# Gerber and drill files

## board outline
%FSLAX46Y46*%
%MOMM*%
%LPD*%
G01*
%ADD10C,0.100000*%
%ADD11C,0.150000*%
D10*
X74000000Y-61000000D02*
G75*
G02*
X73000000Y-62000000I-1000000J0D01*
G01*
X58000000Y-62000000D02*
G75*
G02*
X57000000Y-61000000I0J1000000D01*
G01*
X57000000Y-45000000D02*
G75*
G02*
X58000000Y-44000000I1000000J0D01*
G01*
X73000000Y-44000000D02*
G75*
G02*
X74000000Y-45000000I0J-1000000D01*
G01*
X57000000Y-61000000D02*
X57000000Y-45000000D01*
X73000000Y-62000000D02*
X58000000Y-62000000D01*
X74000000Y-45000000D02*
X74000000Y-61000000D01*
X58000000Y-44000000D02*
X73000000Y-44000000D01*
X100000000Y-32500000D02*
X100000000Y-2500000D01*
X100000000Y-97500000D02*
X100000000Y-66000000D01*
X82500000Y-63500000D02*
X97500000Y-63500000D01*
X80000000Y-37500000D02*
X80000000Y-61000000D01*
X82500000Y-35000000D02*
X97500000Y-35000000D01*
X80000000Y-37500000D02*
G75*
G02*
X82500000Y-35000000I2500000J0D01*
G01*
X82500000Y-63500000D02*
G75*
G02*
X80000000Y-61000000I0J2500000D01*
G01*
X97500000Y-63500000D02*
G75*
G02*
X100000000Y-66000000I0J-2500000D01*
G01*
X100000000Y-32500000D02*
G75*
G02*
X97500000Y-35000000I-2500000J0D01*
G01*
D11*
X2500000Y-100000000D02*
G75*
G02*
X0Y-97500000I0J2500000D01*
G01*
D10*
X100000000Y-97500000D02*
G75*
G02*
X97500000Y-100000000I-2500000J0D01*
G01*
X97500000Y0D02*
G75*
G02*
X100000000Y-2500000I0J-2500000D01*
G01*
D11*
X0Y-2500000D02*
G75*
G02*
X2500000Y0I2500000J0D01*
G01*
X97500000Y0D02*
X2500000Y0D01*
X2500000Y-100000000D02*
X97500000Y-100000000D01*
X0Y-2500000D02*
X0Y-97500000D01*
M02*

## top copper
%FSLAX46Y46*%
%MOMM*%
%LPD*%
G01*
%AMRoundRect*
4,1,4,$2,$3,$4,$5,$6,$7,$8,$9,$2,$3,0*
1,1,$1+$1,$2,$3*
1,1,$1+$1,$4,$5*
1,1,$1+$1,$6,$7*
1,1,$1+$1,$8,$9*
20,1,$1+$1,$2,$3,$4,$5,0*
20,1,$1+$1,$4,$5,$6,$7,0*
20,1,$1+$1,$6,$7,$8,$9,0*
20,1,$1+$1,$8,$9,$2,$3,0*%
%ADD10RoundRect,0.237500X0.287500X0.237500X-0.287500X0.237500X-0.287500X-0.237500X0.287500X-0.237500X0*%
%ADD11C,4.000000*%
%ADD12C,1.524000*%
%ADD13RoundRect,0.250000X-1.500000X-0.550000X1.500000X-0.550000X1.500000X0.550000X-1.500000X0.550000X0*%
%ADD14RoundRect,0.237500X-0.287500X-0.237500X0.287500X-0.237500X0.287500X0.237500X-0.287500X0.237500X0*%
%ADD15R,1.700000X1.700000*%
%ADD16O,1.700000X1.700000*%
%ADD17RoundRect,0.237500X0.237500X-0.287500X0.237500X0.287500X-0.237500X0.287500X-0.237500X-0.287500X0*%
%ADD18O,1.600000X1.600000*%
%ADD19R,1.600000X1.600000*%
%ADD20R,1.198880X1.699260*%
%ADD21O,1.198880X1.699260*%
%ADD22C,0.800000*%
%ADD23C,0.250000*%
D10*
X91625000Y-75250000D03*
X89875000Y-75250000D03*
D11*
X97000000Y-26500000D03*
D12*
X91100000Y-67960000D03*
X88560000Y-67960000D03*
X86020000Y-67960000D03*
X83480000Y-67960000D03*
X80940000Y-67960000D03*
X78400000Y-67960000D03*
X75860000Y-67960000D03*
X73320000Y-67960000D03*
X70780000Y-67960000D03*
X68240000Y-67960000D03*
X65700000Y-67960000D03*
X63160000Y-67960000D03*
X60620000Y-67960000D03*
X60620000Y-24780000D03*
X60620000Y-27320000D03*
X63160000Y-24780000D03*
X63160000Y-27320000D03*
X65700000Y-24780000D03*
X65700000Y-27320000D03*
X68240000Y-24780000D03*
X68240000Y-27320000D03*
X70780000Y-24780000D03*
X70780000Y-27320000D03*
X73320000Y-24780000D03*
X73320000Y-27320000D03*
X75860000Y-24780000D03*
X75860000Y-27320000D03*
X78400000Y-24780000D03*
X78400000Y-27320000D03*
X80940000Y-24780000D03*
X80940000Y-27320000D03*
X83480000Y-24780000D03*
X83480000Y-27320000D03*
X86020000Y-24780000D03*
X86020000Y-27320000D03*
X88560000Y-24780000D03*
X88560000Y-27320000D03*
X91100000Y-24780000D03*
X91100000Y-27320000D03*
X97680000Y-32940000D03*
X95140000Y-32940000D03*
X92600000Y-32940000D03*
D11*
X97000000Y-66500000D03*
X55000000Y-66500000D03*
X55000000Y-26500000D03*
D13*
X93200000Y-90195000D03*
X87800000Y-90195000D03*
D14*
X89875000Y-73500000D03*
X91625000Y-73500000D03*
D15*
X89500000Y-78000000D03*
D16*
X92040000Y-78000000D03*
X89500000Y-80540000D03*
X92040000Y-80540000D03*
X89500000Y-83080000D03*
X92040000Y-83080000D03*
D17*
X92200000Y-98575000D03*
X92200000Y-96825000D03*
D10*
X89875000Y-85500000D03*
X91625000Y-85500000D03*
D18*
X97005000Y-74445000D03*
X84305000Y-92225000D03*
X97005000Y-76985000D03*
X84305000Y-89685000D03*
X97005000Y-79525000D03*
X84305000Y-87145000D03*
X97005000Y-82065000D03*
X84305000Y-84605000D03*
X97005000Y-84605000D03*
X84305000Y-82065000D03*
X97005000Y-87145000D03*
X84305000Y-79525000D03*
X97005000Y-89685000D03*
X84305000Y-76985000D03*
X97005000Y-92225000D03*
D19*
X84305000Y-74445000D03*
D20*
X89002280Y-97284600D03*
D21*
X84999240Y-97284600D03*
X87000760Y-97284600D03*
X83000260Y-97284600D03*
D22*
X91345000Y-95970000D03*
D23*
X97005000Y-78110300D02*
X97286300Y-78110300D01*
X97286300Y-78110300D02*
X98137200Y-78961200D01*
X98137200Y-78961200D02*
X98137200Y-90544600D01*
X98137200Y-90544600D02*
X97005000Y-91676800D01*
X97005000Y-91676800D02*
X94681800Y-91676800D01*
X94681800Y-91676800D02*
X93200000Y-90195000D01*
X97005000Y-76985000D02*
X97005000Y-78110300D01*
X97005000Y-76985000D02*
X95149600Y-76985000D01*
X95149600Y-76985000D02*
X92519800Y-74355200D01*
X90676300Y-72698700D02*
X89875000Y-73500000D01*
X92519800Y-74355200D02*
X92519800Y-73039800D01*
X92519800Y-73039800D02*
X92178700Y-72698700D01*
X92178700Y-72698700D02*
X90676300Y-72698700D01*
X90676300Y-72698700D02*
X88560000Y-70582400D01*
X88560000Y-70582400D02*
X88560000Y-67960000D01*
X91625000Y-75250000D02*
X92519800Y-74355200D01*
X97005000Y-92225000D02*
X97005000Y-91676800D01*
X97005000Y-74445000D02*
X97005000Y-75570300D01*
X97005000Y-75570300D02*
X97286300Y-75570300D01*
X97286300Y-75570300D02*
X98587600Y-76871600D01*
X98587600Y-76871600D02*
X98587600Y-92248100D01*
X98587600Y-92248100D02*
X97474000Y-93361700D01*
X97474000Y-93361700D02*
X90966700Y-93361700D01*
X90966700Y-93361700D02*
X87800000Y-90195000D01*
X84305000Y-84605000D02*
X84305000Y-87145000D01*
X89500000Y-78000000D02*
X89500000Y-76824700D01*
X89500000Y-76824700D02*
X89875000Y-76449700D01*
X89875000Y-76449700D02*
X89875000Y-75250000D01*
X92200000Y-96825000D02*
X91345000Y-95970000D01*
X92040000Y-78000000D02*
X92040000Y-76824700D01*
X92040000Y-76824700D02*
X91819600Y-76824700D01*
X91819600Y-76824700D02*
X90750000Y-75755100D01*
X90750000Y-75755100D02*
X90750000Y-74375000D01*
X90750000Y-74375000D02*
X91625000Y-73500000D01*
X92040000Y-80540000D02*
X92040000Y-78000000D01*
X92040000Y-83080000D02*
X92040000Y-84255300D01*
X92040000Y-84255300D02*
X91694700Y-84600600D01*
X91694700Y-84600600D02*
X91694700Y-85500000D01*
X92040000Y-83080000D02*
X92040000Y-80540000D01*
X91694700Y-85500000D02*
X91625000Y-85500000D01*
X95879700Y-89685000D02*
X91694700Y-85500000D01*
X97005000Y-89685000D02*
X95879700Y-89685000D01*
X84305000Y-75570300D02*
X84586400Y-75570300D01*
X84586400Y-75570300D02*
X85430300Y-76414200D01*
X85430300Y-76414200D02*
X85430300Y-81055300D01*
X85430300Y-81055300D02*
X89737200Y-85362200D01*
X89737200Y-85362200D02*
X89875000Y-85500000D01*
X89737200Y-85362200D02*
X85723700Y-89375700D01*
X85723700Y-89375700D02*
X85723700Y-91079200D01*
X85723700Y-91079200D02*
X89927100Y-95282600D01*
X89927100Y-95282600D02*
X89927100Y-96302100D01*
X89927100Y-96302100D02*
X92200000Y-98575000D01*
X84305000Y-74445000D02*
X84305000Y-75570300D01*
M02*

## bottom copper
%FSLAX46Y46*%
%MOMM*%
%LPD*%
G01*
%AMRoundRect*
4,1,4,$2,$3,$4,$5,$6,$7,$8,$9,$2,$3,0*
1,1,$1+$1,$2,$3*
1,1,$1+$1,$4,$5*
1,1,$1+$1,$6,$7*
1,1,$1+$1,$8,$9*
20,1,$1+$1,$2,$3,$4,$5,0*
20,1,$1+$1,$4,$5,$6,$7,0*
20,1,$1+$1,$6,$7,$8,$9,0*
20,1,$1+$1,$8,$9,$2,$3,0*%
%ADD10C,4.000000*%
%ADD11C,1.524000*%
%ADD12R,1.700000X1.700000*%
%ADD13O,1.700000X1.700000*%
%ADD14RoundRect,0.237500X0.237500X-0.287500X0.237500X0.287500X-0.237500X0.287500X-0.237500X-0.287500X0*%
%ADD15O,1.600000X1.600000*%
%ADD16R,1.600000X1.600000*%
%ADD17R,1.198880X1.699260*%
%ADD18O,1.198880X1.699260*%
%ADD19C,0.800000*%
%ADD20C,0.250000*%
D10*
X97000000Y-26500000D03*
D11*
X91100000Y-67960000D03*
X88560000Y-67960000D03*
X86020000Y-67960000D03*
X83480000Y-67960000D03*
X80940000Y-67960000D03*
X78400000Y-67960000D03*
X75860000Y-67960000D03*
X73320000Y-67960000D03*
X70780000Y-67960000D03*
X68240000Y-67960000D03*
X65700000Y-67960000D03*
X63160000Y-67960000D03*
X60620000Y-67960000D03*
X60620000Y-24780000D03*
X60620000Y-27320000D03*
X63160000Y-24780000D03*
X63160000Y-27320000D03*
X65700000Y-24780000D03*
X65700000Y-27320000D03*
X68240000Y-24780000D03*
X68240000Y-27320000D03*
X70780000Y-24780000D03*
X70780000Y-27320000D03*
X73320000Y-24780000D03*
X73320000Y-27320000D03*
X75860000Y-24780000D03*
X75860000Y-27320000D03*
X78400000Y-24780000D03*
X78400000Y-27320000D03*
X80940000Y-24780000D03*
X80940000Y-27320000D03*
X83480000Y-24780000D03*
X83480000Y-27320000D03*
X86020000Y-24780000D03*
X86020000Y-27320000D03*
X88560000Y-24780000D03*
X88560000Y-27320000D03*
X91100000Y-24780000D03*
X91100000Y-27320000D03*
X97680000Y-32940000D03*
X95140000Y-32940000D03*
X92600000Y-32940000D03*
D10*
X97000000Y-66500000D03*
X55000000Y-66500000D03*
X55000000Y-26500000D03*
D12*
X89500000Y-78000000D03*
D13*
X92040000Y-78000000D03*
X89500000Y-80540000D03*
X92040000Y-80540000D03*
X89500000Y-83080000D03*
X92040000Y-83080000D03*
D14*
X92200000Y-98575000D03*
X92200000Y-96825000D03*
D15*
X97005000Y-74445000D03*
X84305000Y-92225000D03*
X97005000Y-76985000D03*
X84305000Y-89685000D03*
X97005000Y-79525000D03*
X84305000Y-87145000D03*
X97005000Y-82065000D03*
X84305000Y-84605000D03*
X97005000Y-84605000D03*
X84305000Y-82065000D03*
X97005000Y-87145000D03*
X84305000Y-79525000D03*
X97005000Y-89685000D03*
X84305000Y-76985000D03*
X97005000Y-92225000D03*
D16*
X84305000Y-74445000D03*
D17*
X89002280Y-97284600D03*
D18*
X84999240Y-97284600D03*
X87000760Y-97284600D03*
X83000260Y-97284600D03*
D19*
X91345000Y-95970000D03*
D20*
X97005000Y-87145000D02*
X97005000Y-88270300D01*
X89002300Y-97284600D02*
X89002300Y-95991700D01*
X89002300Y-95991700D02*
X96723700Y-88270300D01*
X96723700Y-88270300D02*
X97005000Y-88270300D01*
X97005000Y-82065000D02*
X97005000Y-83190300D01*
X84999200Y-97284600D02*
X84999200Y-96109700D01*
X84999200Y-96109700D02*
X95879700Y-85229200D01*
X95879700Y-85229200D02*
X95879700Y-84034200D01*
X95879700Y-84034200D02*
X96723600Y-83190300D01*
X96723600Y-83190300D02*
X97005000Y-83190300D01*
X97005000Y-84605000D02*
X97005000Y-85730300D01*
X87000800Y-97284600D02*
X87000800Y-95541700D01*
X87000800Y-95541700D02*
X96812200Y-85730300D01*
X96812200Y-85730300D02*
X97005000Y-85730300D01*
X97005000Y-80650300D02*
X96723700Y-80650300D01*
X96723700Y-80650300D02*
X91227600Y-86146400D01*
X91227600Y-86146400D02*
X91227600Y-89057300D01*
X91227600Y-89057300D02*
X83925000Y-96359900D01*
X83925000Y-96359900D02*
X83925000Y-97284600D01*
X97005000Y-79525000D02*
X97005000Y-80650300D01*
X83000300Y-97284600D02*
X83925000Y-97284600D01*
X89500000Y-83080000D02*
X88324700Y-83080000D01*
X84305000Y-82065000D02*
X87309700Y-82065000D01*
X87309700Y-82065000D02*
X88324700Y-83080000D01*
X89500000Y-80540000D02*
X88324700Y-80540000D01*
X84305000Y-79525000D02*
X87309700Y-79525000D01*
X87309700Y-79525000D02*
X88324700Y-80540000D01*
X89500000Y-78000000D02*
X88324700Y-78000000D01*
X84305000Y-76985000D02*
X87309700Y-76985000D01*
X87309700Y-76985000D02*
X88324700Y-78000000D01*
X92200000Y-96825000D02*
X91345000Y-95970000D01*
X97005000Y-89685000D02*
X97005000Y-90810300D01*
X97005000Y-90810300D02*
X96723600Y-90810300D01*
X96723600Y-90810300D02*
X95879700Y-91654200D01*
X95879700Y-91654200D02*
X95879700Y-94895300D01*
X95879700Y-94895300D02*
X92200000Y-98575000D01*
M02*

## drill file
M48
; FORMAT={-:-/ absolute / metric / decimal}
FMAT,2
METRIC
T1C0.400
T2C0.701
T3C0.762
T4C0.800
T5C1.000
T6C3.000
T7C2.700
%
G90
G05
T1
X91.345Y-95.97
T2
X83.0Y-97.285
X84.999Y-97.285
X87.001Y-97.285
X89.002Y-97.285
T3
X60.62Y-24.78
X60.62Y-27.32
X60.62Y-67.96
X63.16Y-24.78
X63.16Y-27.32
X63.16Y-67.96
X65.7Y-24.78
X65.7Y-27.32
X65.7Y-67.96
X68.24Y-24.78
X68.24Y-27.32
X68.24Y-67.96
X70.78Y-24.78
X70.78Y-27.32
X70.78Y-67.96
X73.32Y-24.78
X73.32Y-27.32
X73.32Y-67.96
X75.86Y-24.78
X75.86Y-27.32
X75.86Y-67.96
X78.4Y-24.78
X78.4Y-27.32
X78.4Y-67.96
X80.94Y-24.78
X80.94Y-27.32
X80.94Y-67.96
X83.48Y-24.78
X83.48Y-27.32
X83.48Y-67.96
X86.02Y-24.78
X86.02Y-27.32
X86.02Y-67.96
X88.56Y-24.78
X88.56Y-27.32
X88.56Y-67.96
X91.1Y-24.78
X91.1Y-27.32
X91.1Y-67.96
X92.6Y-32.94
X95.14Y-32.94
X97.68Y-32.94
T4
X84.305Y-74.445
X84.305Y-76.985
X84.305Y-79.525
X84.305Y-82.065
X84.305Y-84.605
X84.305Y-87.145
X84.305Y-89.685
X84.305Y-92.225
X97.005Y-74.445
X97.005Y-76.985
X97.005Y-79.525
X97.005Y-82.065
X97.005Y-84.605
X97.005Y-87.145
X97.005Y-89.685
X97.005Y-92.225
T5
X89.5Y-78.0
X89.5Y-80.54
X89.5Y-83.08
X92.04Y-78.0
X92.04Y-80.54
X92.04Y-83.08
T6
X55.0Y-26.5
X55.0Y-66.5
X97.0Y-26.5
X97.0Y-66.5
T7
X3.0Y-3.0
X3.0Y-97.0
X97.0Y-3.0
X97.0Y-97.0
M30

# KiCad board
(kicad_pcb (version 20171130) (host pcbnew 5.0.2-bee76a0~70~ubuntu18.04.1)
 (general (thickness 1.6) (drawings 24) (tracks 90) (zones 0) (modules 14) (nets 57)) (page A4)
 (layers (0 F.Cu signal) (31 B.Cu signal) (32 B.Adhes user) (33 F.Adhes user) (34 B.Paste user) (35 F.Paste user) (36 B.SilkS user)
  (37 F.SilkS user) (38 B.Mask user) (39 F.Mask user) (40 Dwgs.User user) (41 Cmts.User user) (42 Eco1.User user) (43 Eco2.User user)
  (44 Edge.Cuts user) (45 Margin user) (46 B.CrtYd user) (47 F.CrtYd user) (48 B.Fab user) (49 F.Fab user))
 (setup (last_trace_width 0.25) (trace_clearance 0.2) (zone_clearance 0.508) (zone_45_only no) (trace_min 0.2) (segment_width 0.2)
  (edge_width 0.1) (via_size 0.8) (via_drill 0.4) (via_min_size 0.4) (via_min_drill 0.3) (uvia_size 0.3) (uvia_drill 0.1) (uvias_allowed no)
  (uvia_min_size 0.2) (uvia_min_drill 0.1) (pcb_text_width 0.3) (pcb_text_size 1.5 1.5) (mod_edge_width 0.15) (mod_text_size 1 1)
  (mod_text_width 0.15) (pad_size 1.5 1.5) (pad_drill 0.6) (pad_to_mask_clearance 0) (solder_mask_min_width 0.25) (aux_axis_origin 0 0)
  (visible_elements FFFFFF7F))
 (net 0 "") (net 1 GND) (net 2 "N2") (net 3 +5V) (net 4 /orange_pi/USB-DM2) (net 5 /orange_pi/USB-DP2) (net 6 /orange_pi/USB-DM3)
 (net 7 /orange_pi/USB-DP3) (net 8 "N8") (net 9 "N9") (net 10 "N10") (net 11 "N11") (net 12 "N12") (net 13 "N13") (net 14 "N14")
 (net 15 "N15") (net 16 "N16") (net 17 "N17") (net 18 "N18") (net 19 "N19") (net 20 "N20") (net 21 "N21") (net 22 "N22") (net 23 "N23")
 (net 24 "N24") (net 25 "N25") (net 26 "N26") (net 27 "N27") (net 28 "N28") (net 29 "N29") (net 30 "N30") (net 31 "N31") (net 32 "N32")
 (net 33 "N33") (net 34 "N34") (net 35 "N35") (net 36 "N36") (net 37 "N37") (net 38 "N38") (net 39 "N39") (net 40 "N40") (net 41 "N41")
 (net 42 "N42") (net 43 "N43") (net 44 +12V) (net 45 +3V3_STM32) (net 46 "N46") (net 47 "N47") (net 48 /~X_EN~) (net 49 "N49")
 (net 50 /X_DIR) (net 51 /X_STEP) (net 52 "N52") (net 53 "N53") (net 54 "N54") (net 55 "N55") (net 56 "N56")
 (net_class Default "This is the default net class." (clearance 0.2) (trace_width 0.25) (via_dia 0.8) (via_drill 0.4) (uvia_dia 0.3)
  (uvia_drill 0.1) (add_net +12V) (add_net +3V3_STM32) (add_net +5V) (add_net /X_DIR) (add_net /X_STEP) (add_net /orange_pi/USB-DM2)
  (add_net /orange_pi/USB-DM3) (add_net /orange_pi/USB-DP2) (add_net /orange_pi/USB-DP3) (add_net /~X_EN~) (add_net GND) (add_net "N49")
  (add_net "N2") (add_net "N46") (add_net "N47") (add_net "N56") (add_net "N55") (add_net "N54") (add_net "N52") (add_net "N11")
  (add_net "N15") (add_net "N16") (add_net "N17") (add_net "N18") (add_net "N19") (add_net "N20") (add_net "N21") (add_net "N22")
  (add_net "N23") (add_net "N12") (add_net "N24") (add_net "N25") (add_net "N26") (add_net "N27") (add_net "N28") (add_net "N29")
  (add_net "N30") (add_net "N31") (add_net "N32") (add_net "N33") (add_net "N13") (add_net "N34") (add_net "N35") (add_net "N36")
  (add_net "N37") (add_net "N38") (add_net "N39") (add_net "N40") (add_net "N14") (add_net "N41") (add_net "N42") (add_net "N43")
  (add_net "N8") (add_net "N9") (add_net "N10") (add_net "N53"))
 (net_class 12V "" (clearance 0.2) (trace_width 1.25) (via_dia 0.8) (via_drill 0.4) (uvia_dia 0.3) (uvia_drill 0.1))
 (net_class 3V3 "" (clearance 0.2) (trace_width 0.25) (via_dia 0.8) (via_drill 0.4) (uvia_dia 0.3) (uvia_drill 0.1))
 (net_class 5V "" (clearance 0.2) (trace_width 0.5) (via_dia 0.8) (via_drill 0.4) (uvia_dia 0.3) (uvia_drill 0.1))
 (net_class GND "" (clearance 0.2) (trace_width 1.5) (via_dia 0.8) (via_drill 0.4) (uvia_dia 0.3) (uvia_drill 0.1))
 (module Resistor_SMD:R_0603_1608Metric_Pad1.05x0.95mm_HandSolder (layer F.Cu) (at 90.75 75.25 180)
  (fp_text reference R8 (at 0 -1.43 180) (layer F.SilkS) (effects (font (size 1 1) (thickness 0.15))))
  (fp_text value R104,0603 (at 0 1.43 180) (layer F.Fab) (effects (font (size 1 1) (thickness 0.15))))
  (pad 1 smd roundrect (at -0.875 0 180) (size 1.05 0.95) (layers F.Cu F.Paste F.Mask) (roundrect_rratio 0.25) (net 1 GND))
  (pad 2 smd roundrect (at 0.875 0 180) (size 1.05 0.95) (layers F.Cu F.Paste F.Mask) (roundrect_rratio 0.25) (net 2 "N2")))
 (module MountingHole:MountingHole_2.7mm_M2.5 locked (layer F.Cu) (at 3 97)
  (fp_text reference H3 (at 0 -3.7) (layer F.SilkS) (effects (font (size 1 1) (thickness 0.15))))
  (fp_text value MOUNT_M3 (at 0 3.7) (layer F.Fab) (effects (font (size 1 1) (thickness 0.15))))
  (pad 1 np_thru_hole circle (at 0 0) (size 2.7 2.7) (drill 2.7) (layers *.Cu *.Mask)))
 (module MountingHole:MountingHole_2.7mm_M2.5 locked (layer F.Cu) (at 97 97)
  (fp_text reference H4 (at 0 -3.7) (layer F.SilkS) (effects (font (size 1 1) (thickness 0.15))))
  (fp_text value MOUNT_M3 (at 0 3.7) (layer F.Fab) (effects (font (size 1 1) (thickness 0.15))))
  (pad 1 np_thru_hole circle (at 0 0) (size 2.7 2.7) (drill 2.7) (layers *.Cu *.Mask)))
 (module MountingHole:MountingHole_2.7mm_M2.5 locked (layer F.Cu) (at 3 3)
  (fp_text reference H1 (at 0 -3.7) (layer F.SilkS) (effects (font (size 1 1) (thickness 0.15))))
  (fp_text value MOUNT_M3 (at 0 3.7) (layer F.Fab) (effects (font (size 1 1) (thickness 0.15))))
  (pad 1 np_thru_hole circle (at 0 0) (size 2.7 2.7) (drill 2.7) (layers *.Cu *.Mask)))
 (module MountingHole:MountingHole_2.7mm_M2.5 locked (layer F.Cu) (at 97 3)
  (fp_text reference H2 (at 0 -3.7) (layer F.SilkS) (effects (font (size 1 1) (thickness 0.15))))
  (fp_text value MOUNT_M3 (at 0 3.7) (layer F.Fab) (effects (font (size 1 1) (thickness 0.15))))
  (pad 1 np_thru_hole circle (at 0 0) (size 2.7 2.7) (drill 2.7) (layers *.Cu *.Mask)))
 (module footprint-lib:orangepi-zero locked (layer B.Cu) (at 52 69.5 90)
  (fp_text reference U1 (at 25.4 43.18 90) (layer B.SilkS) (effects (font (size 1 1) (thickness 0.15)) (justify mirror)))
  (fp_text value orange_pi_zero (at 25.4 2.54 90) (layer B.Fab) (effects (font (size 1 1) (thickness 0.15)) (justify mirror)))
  (pad "" thru_hole circle (at 43 45 90) (size 4 4) (drill 3) (layers *.Cu *.Mask B.SilkS))
  (pad 1 thru_hole circle (at 1.54 39.1 90) (size 1.524 1.524) (drill 0.762) (layers *.Cu *.Mask B.SilkS) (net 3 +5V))
  (pad 2 thru_hole circle (at 1.54 36.56 90) (size 1.524 1.524) (drill 0.762) (layers *.Cu *.Mask B.SilkS) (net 1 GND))
  (pad 3 thru_hole circle (at 1.54 34.02 90) (size 1.524 1.524) (drill 0.762) (layers *.Cu *.Mask B.SilkS) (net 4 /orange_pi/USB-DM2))
  (pad 4 thru_hole circle (at 1.54 31.48 90) (size 1.524 1.524) (drill 0.762) (layers *.Cu *.Mask B.SilkS) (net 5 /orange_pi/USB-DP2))
  (pad 5 thru_hole circle (at 1.54 28.94 90) (size 1.524 1.524) (drill 0.762) (layers *.Cu *.Mask B.SilkS) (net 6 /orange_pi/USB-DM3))
  (pad 6 thru_hole circle (at 1.54 26.4 90) (size 1.524 1.524) (drill 0.762) (layers *.Cu *.Mask B.SilkS) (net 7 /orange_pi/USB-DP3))
  (pad 7 thru_hole circle (at 1.54 23.86 90) (size 1.524 1.524) (drill 0.762) (layers *.Cu *.Mask B.SilkS) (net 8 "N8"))
  (pad 8 thru_hole circle (at 1.54 21.32 90) (size 1.524 1.524) (drill 0.762) (layers *.Cu *.Mask B.SilkS) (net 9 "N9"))
  (pad 9 thru_hole circle (at 1.54 18.78 90) (size 1.524 1.524) (drill 0.762) (layers *.Cu *.Mask B.SilkS) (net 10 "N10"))
  (pad 10 thru_hole circle (at 1.54 16.24 90) (size 1.524 1.524) (drill 0.762) (layers *.Cu *.Mask B.SilkS) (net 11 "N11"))
  (pad 11 thru_hole circle (at 1.54 13.7 90) (size 1.524 1.524) (drill 0.762) (layers *.Cu *.Mask B.SilkS) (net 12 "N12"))
  (pad 12 thru_hole circle (at 1.54 11.16 90) (size 1.524 1.524) (drill 0.762) (layers *.Cu *.Mask B.SilkS) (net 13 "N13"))
  (pad 13 thru_hole circle (at 1.54 8.62 90) (size 1.524 1.524) (drill 0.762) (layers *.Cu *.Mask B.SilkS) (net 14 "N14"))
  (pad 101 thru_hole circle (at 44.72 8.62 90) (size 1.524 1.524) (drill 0.762) (layers *.Cu *.Mask B.SilkS) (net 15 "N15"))
  (pad 102 thru_hole circle (at 42.18 8.62 90) (size 1.524 1.524) (drill 0.762) (layers *.Cu *.Mask B.SilkS) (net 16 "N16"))
  (pad 103 thru_hole circle (at 44.72 11.16 90) (size 1.524 1.524) (drill 0.762) (layers *.Cu *.Mask B.SilkS) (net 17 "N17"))
  (pad 104 thru_hole circle (at 42.18 11.16 90) (size 1.524 1.524) (drill 0.762) (layers *.Cu *.Mask B.SilkS) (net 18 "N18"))
  (pad 105 thru_hole circle (at 44.72 13.7 90) (size 1.524 1.524) (drill 0.762) (layers *.Cu *.Mask B.SilkS) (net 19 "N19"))
  (pad 106 thru_hole circle (at 42.18 13.7 90) (size 1.524 1.524) (drill 0.762) (layers *.Cu *.Mask B.SilkS) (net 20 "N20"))
  (pad 107 thru_hole circle (at 44.72 16.24 90) (size 1.524 1.524) (drill 0.762) (layers *.Cu *.Mask B.SilkS) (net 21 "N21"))
  (pad 108 thru_hole circle (at 42.18 16.24 90) (size 1.524 1.524) (drill 0.762) (layers *.Cu *.Mask B.SilkS) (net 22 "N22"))
  (pad 109 thru_hole circle (at 44.72 18.78 90) (size 1.524 1.524) (drill 0.762) (layers *.Cu *.Mask B.SilkS) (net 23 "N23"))
  (pad 110 thru_hole circle (at 42.18 18.78 90) (size 1.524 1.524) (drill 0.762) (layers *.Cu *.Mask B.SilkS) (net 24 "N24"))
  (pad 111 thru_hole circle (at 44.72 21.32 90) (size 1.524 1.524) (drill 0.762) (layers *.Cu *.Mask B.SilkS) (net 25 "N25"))
  (pad 112 thru_hole circle (at 42.18 21.32 90) (size 1.524 1.524) (drill 0.762) (layers *.Cu *.Mask B.SilkS) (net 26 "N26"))
  (pad 113 thru_hole circle (at 44.72 23.86 90) (size 1.524 1.524) (drill 0.762) (layers *.Cu *.Mask B.SilkS) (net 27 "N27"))
  (pad 114 thru_hole circle (at 42.18 23.86 90) (size 1.524 1.524) (drill 0.762) (layers *.Cu *.Mask B.SilkS) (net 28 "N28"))
  (pad 115 thru_hole circle (at 44.72 26.4 90) (size 1.524 1.524) (drill 0.762) (layers *.Cu *.Mask B.SilkS) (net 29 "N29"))
  (pad 116 thru_hole circle (at 42.18 26.4 90) (size 1.524 1.524) (drill 0.762) (layers *.Cu *.Mask B.SilkS) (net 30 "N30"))
  (pad 117 thru_hole circle (at 44.72 28.94 90) (size 1.524 1.524) (drill 0.762) (layers *.Cu *.Mask B.SilkS) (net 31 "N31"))
  (pad 118 thru_hole circle (at 42.18 28.94 90) (size 1.524 1.524) (drill 0.762) (layers *.Cu *.Mask B.SilkS) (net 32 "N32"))
  (pad 119 thru_hole circle (at 44.72 31.48 90) (size 1.524 1.524) (drill 0.762) (layers *.Cu *.Mask B.SilkS) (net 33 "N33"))
  (pad 120 thru_hole circle (at 42.18 31.48 90) (size 1.524 1.524) (drill 0.762) (layers *.Cu *.Mask B.SilkS) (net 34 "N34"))
  (pad 121 thru_hole circle (at 44.72 34.02 90) (size 1.524 1.524) (drill 0.762) (layers *.Cu *.Mask B.SilkS) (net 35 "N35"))
  (pad 122 thru_hole circle (at 42.18 34.02 90) (size 1.524 1.524) (drill 0.762) (layers *.Cu *.Mask B.SilkS) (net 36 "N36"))
  (pad 123 thru_hole circle (at 44.72 36.56 90) (size 1.524 1.524) (drill 0.762) (layers *.Cu *.Mask B.SilkS) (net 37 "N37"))
  (pad 124 thru_hole circle (at 42.18 36.56 90) (size 1.524 1.524) (drill 0.762) (layers *.Cu *.Mask B.SilkS) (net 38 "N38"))
  (pad 125 thru_hole circle (at 44.72 39.1 90) (size 1.524 1.524) (drill 0.762) (layers *.Cu *.Mask B.SilkS) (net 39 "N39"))
  (pad 126 thru_hole circle (at 42.18 39.1 90) (size 1.524 1.524) (drill 0.762) (layers *.Cu *.Mask B.SilkS) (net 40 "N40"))
  (pad 201 thru_hole circle (at 36.56 45.68 90) (size 1.524 1.524) (drill 0.762) (layers *.Cu *.Mask B.SilkS) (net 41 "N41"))
  (pad 202 thru_hole circle (at 36.56 43.14 90) (size 1.524 1.524) (drill 0.762) (layers *.Cu *.Mask B.SilkS) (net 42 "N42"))
  (pad 203 thru_hole circle (at 36.56 40.6 90) (size 1.524 1.524) (drill 0.762) (layers *.Cu *.Mask B.SilkS) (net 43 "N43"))
  (pad "" thru_hole circle (at 3 45 90) (size 4 4) (drill 3) (layers *.Cu *.Mask B.SilkS))
  (pad "" thru_hole circle (at 3 3 90) (size 4 4) (drill 3) (layers *.Cu *.Mask B.SilkS))
  (pad "" thru_hole circle (at 43 3 90) (size 4 4) (drill 3) (layers *.Cu *.Mask B.SilkS)))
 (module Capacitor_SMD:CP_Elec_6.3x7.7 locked (layer F.Cu) (at 90.5 90.195)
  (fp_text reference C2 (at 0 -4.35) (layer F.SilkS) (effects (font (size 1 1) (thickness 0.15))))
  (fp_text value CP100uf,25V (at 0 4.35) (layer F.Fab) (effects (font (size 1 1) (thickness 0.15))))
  (pad 2 smd roundrect (at 2.7 0) (size 3.5 1.6) (layers F.Cu F.Paste F.Mask) (roundrect_rratio 0.15625) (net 1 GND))
  (pad 1 smd roundrect (at -2.7 0) (size 3.5 1.6) (layers F.Cu F.Paste F.Mask) (roundrect_rratio 0.15625) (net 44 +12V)))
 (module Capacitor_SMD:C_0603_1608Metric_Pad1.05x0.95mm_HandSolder (layer F.Cu) (at 90.75 73.5)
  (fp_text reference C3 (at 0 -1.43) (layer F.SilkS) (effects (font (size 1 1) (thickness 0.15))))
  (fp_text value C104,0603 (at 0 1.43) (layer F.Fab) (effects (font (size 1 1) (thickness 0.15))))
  (pad 1 smd roundrect (at -0.875 0) (size 1.05 0.95) (layers F.Cu F.Paste F.Mask) (roundrect_rratio 0.25) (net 1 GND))
  (pad 2 smd roundrect (at 0.875 0) (size 1.05 0.95) (layers F.Cu F.Paste F.Mask) (roundrect_rratio 0.25) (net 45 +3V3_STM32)))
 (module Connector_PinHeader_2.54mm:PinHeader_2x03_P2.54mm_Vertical (layer F.Cu) (at 89.5 78)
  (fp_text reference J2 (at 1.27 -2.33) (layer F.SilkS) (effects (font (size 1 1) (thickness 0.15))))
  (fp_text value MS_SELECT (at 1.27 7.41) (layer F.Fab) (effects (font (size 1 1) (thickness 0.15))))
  (pad 1 thru_hole rect (at 0 0) (size 1.7 1.7) (drill 1) (layers *.Cu *.Mask) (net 2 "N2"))
  (pad 2 thru_hole oval (at 2.54 0) (size 1.7 1.7) (drill 1) (layers *.Cu *.Mask) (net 45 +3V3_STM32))
  (pad 3 thru_hole oval (at 0 2.54) (size 1.7 1.7) (drill 1) (layers *.Cu *.Mask) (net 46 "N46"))
  (pad 4 thru_hole oval (at 2.54 2.54) (size 1.7 1.7) (drill 1) (layers *.Cu *.Mask) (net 45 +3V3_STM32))
  (pad 5 thru_hole oval (at 0 5.08) (size 1.7 1.7) (drill 1) (layers *.Cu *.Mask) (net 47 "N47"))
  (pad 6 thru_hole oval (at 2.54 5.08) (size 1.7 1.7) (drill 1) (layers *.Cu *.Mask) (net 45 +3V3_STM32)))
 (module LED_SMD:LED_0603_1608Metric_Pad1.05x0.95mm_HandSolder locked (layer F.Cu) (at 92.2 97.7 90)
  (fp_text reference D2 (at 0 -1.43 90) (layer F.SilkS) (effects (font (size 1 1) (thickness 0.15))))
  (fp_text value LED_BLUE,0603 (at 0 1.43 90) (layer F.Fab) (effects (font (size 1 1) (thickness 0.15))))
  (pad 1 smd roundrect (at -0.875 0 90) (size 1.05 0.95) (layers F.Cu F.Paste F.Mask) (roundrect_rratio 0.25) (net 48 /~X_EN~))
  (pad 2 smd roundrect (at 0.875 0 90) (size 1.05 0.95) (layers F.Cu F.Paste F.Mask) (roundrect_rratio 0.25) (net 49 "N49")))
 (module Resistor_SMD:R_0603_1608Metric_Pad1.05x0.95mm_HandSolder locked (layer B.Cu) (at 92.2 97.7 90)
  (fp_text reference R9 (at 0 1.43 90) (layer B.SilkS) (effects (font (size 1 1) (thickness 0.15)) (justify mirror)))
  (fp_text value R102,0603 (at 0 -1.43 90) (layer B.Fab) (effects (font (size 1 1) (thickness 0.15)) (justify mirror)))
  (pad 1 smd roundrect (at -0.875 0 90) (size 1.05 0.95) (layers B.Cu B.Paste B.Mask) (roundrect_rratio 0.25) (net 45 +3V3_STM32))
  (pad 2 smd roundrect (at 0.875 0 90) (size 1.05 0.95) (layers B.Cu B.Paste B.Mask) (roundrect_rratio 0.25) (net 49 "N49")))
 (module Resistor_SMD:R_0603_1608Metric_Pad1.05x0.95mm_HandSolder (layer F.Cu) (at 90.75 85.5 180)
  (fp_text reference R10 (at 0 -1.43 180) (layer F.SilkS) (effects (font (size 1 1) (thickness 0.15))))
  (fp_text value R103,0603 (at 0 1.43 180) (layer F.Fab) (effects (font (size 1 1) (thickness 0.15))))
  (pad 2 smd roundrect (at 0.875 0 180) (size 1.05 0.95) (layers F.Cu F.Paste F.Mask) (roundrect_rratio 0.25) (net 48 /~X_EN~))
  (pad 1 smd roundrect (at -0.875 0 180) (size 1.05 0.95) (layers F.Cu F.Paste F.Mask) (roundrect_rratio 0.25) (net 45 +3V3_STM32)))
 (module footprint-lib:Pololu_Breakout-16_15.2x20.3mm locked (layer F.Cu) (at 84.305 74.445)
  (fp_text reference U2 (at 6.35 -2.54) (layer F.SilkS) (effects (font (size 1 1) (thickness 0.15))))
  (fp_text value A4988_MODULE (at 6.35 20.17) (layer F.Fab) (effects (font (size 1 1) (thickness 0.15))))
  (pad 16 thru_hole oval (at 12.7 0) (size 1.6 1.6) (drill 0.8) (layers *.Cu *.Mask) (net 44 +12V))
  (pad 8 thru_hole oval (at 0 17.78) (size 1.6 1.6) (drill 0.8) (layers *.Cu *.Mask) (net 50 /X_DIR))
  (pad 15 thru_hole oval (at 12.7 2.54) (size 1.6 1.6) (drill 0.8) (layers *.Cu *.Mask) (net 1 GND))
  (pad 7 thru_hole oval (at 0 15.24) (size 1.6 1.6) (drill 0.8) (layers *.Cu *.Mask) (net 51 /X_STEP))
  (pad 14 thru_hole oval (at 12.7 5.08) (size 1.6 1.6) (drill 0.8) (layers *.Cu *.Mask) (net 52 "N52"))
  (pad 6 thru_hole oval (at 0 12.7) (size 1.6 1.6) (drill 0.8) (layers *.Cu *.Mask) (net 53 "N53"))
  (pad 13 thru_hole oval (at 12.7 7.62) (size 1.6 1.6) (drill 0.8) (layers *.Cu *.Mask) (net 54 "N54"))
  (pad 5 thru_hole oval (at 0 10.16) (size 1.6 1.6) (drill 0.8) (layers *.Cu *.Mask) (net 53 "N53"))
  (pad 12 thru_hole oval (at 12.7 10.16) (size 1.6 1.6) (drill 0.8) (layers *.Cu *.Mask) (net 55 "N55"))
  (pad 4 thru_hole oval (at 0 7.62) (size 1.6 1.6) (drill 0.8) (layers *.Cu *.Mask) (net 47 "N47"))
  (pad 11 thru_hole oval (at 12.7 12.7) (size 1.6 1.6) (drill 0.8) (layers *.Cu *.Mask) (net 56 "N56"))
  (pad 3 thru_hole oval (at 0 5.08) (size 1.6 1.6) (drill 0.8) (layers *.Cu *.Mask) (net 46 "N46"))
  (pad 10 thru_hole oval (at 12.7 15.24) (size 1.6 1.6) (drill 0.8) (layers *.Cu *.Mask) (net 45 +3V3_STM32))
  (pad 2 thru_hole oval (at 0 2.54) (size 1.6 1.6) (drill 0.8) (layers *.Cu *.Mask) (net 2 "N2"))
  (pad 9 thru_hole oval (at 12.7 17.78) (size 1.6 1.6) (drill 0.8) (layers *.Cu *.Mask) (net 1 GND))
  (pad 1 thru_hole rect (at 0 0) (size 1.6 1.6) (drill 0.8) (layers *.Cu *.Mask) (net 48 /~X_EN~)))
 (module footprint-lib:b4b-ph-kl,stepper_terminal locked (layer F.Cu) (at 86 97.2846 180)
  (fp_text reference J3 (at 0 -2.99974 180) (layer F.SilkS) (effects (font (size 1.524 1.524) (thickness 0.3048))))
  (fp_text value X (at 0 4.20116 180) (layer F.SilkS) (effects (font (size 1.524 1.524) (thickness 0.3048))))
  (pad 1 thru_hole rect (at -3.00228 0 180) (size 1.19888 1.69926) (drill 0.70104) (layers *.Cu *.Mask F.SilkS) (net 56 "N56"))
  (pad 3 thru_hole oval (at 1.00076 0 180) (size 1.19888 1.69926) (drill 0.70104) (layers *.Cu *.Mask F.SilkS) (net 54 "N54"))
  (pad 2 thru_hole oval (at -1.00076 0 180) (size 1.19888 1.69926) (drill 0.70104) (layers *.Cu *.Mask F.SilkS) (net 55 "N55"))
  (pad 4 thru_hole oval (at 2.99974 0 180) (size 1.19888 1.69926) (drill 0.70104) (layers *.Cu *.Mask F.SilkS) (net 52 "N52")))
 (gr_arc (start 73 61) (end 73 62) (angle -90) (layer Edge.Cuts) (width 0.1))
 (gr_arc (start 58 61) (end 57 61) (angle -90) (layer Edge.Cuts) (width 0.1))
 (gr_arc (start 58 45) (end 58 44) (angle -90) (layer Edge.Cuts) (width 0.1))
 (gr_arc (start 73 45) (end 74 45) (angle -90) (layer Edge.Cuts) (width 0.1))
 (gr_line (start 57 61) (end 57 45) (layer Edge.Cuts) (width 0.1))
 (gr_line (start 73 62) (end 58 62) (layer Edge.Cuts) (width 0.1))
 (gr_line (start 74 45) (end 74 61) (layer Edge.Cuts) (width 0.1))
 (gr_line (start 58 44) (end 73 44) (layer Edge.Cuts) (width 0.1))
 (gr_line (start 100 32.5) (end 100 2.5) (layer Edge.Cuts) (width 0.1))
 (gr_line (start 100 97.5) (end 100 66) (layer Edge.Cuts) (width 0.1))
 (gr_line (start 82.5 63.5) (end 97.5 63.5) (layer Edge.Cuts) (width 0.1))
 (gr_line (start 80 37.5) (end 80 61) (layer Edge.Cuts) (width 0.1))
 (gr_line (start 82.5 35) (end 97.5 35) (layer Edge.Cuts) (width 0.1))
 (gr_arc (start 82.5 37.5) (end 82.5 35) (angle -90) (layer Edge.Cuts) (width 0.1))
 (gr_arc (start 82.5 61) (end 80 61) (angle -90) (layer Edge.Cuts) (width 0.1))
 (gr_arc (start 97.5 66) (end 100 66) (angle -90) (layer Edge.Cuts) (width 0.1))
 (gr_arc (start 97.5 32.5) (end 97.5 35) (angle -90) (layer Edge.Cuts) (width 0.1))
 (gr_arc (start 2.5 97.5) (end 0 97.5) (angle -90) (layer Edge.Cuts) (width 0.15))
 (gr_arc (start 97.5 97.5) (end 97.5 100) (angle -90) (layer Edge.Cuts) (width 0.1))
 (gr_arc (start 97.5 2.5) (end 100 2.5) (angle -90) (layer Edge.Cuts) (width 0.1))
 (gr_arc (start 2.5 2.5) (end 2.5 0) (angle -90) (layer Edge.Cuts) (width 0.15))
 (gr_line (start 97.5 0) (end 2.5 0) (layer Edge.Cuts) (width 0.15))
 (gr_line (start 2.5 100) (end 97.5 100) (layer Edge.Cuts) (width 0.15))
 (gr_line (start 0 2.5) (end 0 97.5) (layer Edge.Cuts) (width 0.15))
 (segment (start 97.005 78.1103) (end 97.2863 78.1103) (width 0.25) (layer F.Cu) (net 1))
 (segment (start 97.2863 78.1103) (end 98.1372 78.9612) (width 0.25) (layer F.Cu) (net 1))
 (segment (start 98.1372 78.9612) (end 98.1372 90.5446) (width 0.25) (layer F.Cu) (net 1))
 (segment (start 98.1372 90.5446) (end 97.005 91.6768) (width 0.25) (layer F.Cu) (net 1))
 (segment (start 97.005 91.6768) (end 94.6818 91.6768) (width 0.25) (layer F.Cu) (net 1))
 (segment (start 94.6818 91.6768) (end 93.2 90.195) (width 0.25) (layer F.Cu) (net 1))
 (segment (start 97.005 76.985) (end 97.005 78.1103) (width 0.25) (layer F.Cu) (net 1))
 (segment (start 97.005 76.985) (end 95.1496 76.985) (width 0.25) (layer F.Cu) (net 1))
 (segment (start 95.1496 76.985) (end 92.5198 74.3552) (width 0.25) (layer F.Cu) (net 1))
 (segment (start 90.6763 72.6987) (end 89.875 73.5) (width 0.25) (layer F.Cu) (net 1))
 (segment (start 92.5198 74.3552) (end 92.5198 73.0398) (width 0.25) (layer F.Cu) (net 1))
 (segment (start 92.5198 73.0398) (end 92.1787 72.6987) (width 0.25) (layer F.Cu) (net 1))
 (segment (start 92.1787 72.6987) (end 90.6763 72.6987) (width 0.25) (layer F.Cu) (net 1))
 (segment (start 90.6763 72.6987) (end 88.56 70.5824) (width 0.25) (layer F.Cu) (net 1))
 (segment (start 88.56 70.5824) (end 88.56 67.96) (width 0.25) (layer F.Cu) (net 1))
 (segment (start 91.625 75.25) (end 92.5198 74.3552) (width 0.25) (layer F.Cu) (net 1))
 (segment (start 97.005 92.225) (end 97.005 91.6768) (width 0.25) (layer F.Cu) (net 1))
 (segment (start 97.005 74.445) (end 97.005 75.5703) (width 0.25) (layer F.Cu) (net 44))
 (segment (start 97.005 75.5703) (end 97.2863 75.5703) (width 0.25) (layer F.Cu) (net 44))
 (segment (start 97.2863 75.5703) (end 98.5876 76.8716) (width 0.25) (layer F.Cu) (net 44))
 (segment (start 98.5876 76.8716) (end 98.5876 92.2481) (width 0.25) (layer F.Cu) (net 44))
 (segment (start 98.5876 92.2481) (end 97.474 93.3617) (width 0.25) (layer F.Cu) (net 44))
 (segment (start 97.474 93.3617) (end 90.9667 93.3617) (width 0.25) (layer F.Cu) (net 44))
 (segment (start 90.9667 93.3617) (end 87.8 90.195) (width 0.25) (layer F.Cu) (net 44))
 (segment (start 97.005 87.145) (end 97.005 88.2703) (width 0.25) (layer B.Cu) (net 56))
 (segment (start 89.0023 97.2846) (end 89.0023 95.9917) (width 0.25) (layer B.Cu) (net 56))
 (segment (start 89.0023 95.9917) (end 96.7237 88.2703) (width 0.25) (layer B.Cu) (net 56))
 (segment (start 96.7237 88.2703) (end 97.005 88.2703) (width 0.25) (layer B.Cu) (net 56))
 (segment (start 97.005 82.065) (end 97.005 83.1903) (width 0.25) (layer B.Cu) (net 54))
 (segment (start 84.9992 97.2846) (end 84.9992 96.1097) (width 0.25) (layer B.Cu) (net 54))
 (segment (start 84.9992 96.1097) (end 95.8797 85.2292) (width 0.25) (layer B.Cu) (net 54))
 (segment (start 95.8797 85.2292) (end 95.8797 84.0342) (width 0.25) (layer B.Cu) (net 54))
 (segment (start 95.8797 84.0342) (end 96.7236 83.1903) (width 0.25) (layer B.Cu) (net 54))
 (segment (start 96.7236 83.1903) (end 97.005 83.1903) (width 0.25) (layer B.Cu) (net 54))
 (segment (start 97.005 84.605) (end 97.005 85.7303) (width 0.25) (layer B.Cu) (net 55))
 (segment (start 87.0008 97.2846) (end 87.0008 95.5417) (width 0.25) (layer B.Cu) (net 55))
 (segment (start 87.0008 95.5417) (end 96.8122 85.7303) (width 0.25) (layer B.Cu) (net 55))
 (segment (start 96.8122 85.7303) (end 97.005 85.7303) (width 0.25) (layer B.Cu) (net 55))
 (segment (start 97.005 80.6503) (end 96.7237 80.6503) (width 0.25) (layer B.Cu) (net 52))
 (segment (start 96.7237 80.6503) (end 91.2276 86.1464) (width 0.25) (layer B.Cu) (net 52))
 (segment (start 91.2276 86.1464) (end 91.2276 89.0573) (width 0.25) (layer B.Cu) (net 52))
 (segment (start 91.2276 89.0573) (end 83.925 96.3599) (width 0.25) (layer B.Cu) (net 52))
 (segment (start 83.925 96.3599) (end 83.925 97.2846) (width 0.25) (layer B.Cu) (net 52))
 (segment (start 97.005 79.525) (end 97.005 80.6503) (width 0.25) (layer B.Cu) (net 52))
 (segment (start 83.0003 97.2846) (end 83.925 97.2846) (width 0.25) (layer B.Cu) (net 52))
 (segment (start 84.305 84.605) (end 84.305 87.145) (width 0.25) (layer F.Cu) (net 53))
 (segment (start 89.5 83.08) (end 88.3247 83.08) (width 0.25) (layer B.Cu) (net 47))
 (segment (start 84.305 82.065) (end 87.3097 82.065) (width 0.25) (layer B.Cu) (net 47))
 (segment (start 87.3097 82.065) (end 88.3247 83.08) (width 0.25) (layer B.Cu) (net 47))
 (segment (start 89.5 80.54) (end 88.3247 80.54) (width 0.25) (layer B.Cu) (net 46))
 (segment (start 84.305 79.525) (end 87.3097 79.525) (width 0.25) (layer B.Cu) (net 46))
 (segment (start 87.3097 79.525) (end 88.3247 80.54) (width 0.25) (layer B.Cu) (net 46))
 (segment (start 89.5 78) (end 88.3247 78) (width 0.25) (layer B.Cu) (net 2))
 (segment (start 84.305 76.985) (end 87.3097 76.985) (width 0.25) (layer B.Cu) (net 2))
 (segment (start 87.3097 76.985) (end 88.3247 78) (width 0.25) (layer B.Cu) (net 2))
 (segment (start 89.5 78) (end 89.5 76.8247) (width 0.25) (layer F.Cu) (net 2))
 (segment (start 89.5 76.8247) (end 89.875 76.4497) (width 0.25) (layer F.Cu) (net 2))
 (segment (start 89.875 76.4497) (end 89.875 75.25) (width 0.25) (layer F.Cu) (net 2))
 (segment (start 92.2 96.825) (end 91.345 95.97) (width 0.25) (layer F.Cu) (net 49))
 (segment (start 92.2 96.825) (end 91.345 95.97) (width 0.25) (layer B.Cu) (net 49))
 (via (at 91.345 95.97) (size 0.8) (layers F.Cu B.Cu) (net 49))
 (segment (start 92.04 78) (end 92.04 76.8247) (width 0.25) (layer F.Cu) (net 45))
 (segment (start 92.04 76.8247) (end 91.8196 76.8247) (width 0.25) (layer F.Cu) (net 45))
 (segment (start 91.8196 76.8247) (end 90.75 75.7551) (width 0.25) (layer F.Cu) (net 45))
 (segment (start 90.75 75.7551) (end 90.75 74.375) (width 0.25) (layer F.Cu) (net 45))
 (segment (start 90.75 74.375) (end 91.625 73.5) (width 0.25) (layer F.Cu) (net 45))
 (segment (start 92.04 80.54) (end 92.04 78) (width 0.25) (layer F.Cu) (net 45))
 (segment (start 97.005 89.685) (end 97.005 90.8103) (width 0.25) (layer B.Cu) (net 45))
 (segment (start 97.005 90.8103) (end 96.7236 90.8103) (width 0.25) (layer B.Cu) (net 45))
 (segment (start 96.7236 90.8103) (end 95.8797 91.6542) (width 0.25) (layer B.Cu) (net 45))
 (segment (start 95.8797 91.6542) (end 95.8797 94.8953) (width 0.25) (layer B.Cu) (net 45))
 (segment (start 95.8797 94.8953) (end 92.2 98.575) (width 0.25) (layer B.Cu) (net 45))
 (segment (start 92.04 83.08) (end 92.04 84.2553) (width 0.25) (layer F.Cu) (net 45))
 (segment (start 92.04 84.2553) (end 91.6947 84.6006) (width 0.25) (layer F.Cu) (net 45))
 (segment (start 91.6947 84.6006) (end 91.6947 85.5) (width 0.25) (layer F.Cu) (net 45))
 (segment (start 92.04 83.08) (end 92.04 80.54) (width 0.25) (layer F.Cu) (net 45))
 (segment (start 91.6947 85.5) (end 91.625 85.5) (width 0.25) (layer F.Cu) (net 45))
 (segment (start 95.8797 89.685) (end 91.6947 85.5) (width 0.25) (layer F.Cu) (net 45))
 (segment (start 97.005 89.685) (end 95.8797 89.685) (width 0.25) (layer F.Cu) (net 45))
 (segment (start 84.305 75.5703) (end 84.5864 75.5703) (width 0.25) (layer F.Cu) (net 48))
 (segment (start 84.5864 75.5703) (end 85.4303 76.4142) (width 0.25) (layer F.Cu) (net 48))
 (segment (start 85.4303 76.4142) (end 85.4303 81.0553) (width 0.25) (layer F.Cu) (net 48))
 (segment (start 85.4303 81.0553) (end 89.7372 85.3622) (width 0.25) (layer F.Cu) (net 48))
 (segment (start 89.7372 85.3622) (end 89.875 85.5) (width 0.25) (layer F.Cu) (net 48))
 (segment (start 89.7372 85.3622) (end 85.7237 89.3757) (width 0.25) (layer F.Cu) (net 48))
 (segment (start 85.7237 89.3757) (end 85.7237 91.0792) (width 0.25) (layer F.Cu) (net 48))
 (segment (start 85.7237 91.0792) (end 89.9271 95.2826) (width 0.25) (layer F.Cu) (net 48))
 (segment (start 89.9271 95.2826) (end 89.9271 96.3021) (width 0.25) (layer F.Cu) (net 48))
 (segment (start 89.9271 96.3021) (end 92.2 98.575) (width 0.25) (layer F.Cu) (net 48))
 (segment (start 84.305 74.445) (end 84.305 75.5703) (width 0.25) (layer F.Cu) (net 48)))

